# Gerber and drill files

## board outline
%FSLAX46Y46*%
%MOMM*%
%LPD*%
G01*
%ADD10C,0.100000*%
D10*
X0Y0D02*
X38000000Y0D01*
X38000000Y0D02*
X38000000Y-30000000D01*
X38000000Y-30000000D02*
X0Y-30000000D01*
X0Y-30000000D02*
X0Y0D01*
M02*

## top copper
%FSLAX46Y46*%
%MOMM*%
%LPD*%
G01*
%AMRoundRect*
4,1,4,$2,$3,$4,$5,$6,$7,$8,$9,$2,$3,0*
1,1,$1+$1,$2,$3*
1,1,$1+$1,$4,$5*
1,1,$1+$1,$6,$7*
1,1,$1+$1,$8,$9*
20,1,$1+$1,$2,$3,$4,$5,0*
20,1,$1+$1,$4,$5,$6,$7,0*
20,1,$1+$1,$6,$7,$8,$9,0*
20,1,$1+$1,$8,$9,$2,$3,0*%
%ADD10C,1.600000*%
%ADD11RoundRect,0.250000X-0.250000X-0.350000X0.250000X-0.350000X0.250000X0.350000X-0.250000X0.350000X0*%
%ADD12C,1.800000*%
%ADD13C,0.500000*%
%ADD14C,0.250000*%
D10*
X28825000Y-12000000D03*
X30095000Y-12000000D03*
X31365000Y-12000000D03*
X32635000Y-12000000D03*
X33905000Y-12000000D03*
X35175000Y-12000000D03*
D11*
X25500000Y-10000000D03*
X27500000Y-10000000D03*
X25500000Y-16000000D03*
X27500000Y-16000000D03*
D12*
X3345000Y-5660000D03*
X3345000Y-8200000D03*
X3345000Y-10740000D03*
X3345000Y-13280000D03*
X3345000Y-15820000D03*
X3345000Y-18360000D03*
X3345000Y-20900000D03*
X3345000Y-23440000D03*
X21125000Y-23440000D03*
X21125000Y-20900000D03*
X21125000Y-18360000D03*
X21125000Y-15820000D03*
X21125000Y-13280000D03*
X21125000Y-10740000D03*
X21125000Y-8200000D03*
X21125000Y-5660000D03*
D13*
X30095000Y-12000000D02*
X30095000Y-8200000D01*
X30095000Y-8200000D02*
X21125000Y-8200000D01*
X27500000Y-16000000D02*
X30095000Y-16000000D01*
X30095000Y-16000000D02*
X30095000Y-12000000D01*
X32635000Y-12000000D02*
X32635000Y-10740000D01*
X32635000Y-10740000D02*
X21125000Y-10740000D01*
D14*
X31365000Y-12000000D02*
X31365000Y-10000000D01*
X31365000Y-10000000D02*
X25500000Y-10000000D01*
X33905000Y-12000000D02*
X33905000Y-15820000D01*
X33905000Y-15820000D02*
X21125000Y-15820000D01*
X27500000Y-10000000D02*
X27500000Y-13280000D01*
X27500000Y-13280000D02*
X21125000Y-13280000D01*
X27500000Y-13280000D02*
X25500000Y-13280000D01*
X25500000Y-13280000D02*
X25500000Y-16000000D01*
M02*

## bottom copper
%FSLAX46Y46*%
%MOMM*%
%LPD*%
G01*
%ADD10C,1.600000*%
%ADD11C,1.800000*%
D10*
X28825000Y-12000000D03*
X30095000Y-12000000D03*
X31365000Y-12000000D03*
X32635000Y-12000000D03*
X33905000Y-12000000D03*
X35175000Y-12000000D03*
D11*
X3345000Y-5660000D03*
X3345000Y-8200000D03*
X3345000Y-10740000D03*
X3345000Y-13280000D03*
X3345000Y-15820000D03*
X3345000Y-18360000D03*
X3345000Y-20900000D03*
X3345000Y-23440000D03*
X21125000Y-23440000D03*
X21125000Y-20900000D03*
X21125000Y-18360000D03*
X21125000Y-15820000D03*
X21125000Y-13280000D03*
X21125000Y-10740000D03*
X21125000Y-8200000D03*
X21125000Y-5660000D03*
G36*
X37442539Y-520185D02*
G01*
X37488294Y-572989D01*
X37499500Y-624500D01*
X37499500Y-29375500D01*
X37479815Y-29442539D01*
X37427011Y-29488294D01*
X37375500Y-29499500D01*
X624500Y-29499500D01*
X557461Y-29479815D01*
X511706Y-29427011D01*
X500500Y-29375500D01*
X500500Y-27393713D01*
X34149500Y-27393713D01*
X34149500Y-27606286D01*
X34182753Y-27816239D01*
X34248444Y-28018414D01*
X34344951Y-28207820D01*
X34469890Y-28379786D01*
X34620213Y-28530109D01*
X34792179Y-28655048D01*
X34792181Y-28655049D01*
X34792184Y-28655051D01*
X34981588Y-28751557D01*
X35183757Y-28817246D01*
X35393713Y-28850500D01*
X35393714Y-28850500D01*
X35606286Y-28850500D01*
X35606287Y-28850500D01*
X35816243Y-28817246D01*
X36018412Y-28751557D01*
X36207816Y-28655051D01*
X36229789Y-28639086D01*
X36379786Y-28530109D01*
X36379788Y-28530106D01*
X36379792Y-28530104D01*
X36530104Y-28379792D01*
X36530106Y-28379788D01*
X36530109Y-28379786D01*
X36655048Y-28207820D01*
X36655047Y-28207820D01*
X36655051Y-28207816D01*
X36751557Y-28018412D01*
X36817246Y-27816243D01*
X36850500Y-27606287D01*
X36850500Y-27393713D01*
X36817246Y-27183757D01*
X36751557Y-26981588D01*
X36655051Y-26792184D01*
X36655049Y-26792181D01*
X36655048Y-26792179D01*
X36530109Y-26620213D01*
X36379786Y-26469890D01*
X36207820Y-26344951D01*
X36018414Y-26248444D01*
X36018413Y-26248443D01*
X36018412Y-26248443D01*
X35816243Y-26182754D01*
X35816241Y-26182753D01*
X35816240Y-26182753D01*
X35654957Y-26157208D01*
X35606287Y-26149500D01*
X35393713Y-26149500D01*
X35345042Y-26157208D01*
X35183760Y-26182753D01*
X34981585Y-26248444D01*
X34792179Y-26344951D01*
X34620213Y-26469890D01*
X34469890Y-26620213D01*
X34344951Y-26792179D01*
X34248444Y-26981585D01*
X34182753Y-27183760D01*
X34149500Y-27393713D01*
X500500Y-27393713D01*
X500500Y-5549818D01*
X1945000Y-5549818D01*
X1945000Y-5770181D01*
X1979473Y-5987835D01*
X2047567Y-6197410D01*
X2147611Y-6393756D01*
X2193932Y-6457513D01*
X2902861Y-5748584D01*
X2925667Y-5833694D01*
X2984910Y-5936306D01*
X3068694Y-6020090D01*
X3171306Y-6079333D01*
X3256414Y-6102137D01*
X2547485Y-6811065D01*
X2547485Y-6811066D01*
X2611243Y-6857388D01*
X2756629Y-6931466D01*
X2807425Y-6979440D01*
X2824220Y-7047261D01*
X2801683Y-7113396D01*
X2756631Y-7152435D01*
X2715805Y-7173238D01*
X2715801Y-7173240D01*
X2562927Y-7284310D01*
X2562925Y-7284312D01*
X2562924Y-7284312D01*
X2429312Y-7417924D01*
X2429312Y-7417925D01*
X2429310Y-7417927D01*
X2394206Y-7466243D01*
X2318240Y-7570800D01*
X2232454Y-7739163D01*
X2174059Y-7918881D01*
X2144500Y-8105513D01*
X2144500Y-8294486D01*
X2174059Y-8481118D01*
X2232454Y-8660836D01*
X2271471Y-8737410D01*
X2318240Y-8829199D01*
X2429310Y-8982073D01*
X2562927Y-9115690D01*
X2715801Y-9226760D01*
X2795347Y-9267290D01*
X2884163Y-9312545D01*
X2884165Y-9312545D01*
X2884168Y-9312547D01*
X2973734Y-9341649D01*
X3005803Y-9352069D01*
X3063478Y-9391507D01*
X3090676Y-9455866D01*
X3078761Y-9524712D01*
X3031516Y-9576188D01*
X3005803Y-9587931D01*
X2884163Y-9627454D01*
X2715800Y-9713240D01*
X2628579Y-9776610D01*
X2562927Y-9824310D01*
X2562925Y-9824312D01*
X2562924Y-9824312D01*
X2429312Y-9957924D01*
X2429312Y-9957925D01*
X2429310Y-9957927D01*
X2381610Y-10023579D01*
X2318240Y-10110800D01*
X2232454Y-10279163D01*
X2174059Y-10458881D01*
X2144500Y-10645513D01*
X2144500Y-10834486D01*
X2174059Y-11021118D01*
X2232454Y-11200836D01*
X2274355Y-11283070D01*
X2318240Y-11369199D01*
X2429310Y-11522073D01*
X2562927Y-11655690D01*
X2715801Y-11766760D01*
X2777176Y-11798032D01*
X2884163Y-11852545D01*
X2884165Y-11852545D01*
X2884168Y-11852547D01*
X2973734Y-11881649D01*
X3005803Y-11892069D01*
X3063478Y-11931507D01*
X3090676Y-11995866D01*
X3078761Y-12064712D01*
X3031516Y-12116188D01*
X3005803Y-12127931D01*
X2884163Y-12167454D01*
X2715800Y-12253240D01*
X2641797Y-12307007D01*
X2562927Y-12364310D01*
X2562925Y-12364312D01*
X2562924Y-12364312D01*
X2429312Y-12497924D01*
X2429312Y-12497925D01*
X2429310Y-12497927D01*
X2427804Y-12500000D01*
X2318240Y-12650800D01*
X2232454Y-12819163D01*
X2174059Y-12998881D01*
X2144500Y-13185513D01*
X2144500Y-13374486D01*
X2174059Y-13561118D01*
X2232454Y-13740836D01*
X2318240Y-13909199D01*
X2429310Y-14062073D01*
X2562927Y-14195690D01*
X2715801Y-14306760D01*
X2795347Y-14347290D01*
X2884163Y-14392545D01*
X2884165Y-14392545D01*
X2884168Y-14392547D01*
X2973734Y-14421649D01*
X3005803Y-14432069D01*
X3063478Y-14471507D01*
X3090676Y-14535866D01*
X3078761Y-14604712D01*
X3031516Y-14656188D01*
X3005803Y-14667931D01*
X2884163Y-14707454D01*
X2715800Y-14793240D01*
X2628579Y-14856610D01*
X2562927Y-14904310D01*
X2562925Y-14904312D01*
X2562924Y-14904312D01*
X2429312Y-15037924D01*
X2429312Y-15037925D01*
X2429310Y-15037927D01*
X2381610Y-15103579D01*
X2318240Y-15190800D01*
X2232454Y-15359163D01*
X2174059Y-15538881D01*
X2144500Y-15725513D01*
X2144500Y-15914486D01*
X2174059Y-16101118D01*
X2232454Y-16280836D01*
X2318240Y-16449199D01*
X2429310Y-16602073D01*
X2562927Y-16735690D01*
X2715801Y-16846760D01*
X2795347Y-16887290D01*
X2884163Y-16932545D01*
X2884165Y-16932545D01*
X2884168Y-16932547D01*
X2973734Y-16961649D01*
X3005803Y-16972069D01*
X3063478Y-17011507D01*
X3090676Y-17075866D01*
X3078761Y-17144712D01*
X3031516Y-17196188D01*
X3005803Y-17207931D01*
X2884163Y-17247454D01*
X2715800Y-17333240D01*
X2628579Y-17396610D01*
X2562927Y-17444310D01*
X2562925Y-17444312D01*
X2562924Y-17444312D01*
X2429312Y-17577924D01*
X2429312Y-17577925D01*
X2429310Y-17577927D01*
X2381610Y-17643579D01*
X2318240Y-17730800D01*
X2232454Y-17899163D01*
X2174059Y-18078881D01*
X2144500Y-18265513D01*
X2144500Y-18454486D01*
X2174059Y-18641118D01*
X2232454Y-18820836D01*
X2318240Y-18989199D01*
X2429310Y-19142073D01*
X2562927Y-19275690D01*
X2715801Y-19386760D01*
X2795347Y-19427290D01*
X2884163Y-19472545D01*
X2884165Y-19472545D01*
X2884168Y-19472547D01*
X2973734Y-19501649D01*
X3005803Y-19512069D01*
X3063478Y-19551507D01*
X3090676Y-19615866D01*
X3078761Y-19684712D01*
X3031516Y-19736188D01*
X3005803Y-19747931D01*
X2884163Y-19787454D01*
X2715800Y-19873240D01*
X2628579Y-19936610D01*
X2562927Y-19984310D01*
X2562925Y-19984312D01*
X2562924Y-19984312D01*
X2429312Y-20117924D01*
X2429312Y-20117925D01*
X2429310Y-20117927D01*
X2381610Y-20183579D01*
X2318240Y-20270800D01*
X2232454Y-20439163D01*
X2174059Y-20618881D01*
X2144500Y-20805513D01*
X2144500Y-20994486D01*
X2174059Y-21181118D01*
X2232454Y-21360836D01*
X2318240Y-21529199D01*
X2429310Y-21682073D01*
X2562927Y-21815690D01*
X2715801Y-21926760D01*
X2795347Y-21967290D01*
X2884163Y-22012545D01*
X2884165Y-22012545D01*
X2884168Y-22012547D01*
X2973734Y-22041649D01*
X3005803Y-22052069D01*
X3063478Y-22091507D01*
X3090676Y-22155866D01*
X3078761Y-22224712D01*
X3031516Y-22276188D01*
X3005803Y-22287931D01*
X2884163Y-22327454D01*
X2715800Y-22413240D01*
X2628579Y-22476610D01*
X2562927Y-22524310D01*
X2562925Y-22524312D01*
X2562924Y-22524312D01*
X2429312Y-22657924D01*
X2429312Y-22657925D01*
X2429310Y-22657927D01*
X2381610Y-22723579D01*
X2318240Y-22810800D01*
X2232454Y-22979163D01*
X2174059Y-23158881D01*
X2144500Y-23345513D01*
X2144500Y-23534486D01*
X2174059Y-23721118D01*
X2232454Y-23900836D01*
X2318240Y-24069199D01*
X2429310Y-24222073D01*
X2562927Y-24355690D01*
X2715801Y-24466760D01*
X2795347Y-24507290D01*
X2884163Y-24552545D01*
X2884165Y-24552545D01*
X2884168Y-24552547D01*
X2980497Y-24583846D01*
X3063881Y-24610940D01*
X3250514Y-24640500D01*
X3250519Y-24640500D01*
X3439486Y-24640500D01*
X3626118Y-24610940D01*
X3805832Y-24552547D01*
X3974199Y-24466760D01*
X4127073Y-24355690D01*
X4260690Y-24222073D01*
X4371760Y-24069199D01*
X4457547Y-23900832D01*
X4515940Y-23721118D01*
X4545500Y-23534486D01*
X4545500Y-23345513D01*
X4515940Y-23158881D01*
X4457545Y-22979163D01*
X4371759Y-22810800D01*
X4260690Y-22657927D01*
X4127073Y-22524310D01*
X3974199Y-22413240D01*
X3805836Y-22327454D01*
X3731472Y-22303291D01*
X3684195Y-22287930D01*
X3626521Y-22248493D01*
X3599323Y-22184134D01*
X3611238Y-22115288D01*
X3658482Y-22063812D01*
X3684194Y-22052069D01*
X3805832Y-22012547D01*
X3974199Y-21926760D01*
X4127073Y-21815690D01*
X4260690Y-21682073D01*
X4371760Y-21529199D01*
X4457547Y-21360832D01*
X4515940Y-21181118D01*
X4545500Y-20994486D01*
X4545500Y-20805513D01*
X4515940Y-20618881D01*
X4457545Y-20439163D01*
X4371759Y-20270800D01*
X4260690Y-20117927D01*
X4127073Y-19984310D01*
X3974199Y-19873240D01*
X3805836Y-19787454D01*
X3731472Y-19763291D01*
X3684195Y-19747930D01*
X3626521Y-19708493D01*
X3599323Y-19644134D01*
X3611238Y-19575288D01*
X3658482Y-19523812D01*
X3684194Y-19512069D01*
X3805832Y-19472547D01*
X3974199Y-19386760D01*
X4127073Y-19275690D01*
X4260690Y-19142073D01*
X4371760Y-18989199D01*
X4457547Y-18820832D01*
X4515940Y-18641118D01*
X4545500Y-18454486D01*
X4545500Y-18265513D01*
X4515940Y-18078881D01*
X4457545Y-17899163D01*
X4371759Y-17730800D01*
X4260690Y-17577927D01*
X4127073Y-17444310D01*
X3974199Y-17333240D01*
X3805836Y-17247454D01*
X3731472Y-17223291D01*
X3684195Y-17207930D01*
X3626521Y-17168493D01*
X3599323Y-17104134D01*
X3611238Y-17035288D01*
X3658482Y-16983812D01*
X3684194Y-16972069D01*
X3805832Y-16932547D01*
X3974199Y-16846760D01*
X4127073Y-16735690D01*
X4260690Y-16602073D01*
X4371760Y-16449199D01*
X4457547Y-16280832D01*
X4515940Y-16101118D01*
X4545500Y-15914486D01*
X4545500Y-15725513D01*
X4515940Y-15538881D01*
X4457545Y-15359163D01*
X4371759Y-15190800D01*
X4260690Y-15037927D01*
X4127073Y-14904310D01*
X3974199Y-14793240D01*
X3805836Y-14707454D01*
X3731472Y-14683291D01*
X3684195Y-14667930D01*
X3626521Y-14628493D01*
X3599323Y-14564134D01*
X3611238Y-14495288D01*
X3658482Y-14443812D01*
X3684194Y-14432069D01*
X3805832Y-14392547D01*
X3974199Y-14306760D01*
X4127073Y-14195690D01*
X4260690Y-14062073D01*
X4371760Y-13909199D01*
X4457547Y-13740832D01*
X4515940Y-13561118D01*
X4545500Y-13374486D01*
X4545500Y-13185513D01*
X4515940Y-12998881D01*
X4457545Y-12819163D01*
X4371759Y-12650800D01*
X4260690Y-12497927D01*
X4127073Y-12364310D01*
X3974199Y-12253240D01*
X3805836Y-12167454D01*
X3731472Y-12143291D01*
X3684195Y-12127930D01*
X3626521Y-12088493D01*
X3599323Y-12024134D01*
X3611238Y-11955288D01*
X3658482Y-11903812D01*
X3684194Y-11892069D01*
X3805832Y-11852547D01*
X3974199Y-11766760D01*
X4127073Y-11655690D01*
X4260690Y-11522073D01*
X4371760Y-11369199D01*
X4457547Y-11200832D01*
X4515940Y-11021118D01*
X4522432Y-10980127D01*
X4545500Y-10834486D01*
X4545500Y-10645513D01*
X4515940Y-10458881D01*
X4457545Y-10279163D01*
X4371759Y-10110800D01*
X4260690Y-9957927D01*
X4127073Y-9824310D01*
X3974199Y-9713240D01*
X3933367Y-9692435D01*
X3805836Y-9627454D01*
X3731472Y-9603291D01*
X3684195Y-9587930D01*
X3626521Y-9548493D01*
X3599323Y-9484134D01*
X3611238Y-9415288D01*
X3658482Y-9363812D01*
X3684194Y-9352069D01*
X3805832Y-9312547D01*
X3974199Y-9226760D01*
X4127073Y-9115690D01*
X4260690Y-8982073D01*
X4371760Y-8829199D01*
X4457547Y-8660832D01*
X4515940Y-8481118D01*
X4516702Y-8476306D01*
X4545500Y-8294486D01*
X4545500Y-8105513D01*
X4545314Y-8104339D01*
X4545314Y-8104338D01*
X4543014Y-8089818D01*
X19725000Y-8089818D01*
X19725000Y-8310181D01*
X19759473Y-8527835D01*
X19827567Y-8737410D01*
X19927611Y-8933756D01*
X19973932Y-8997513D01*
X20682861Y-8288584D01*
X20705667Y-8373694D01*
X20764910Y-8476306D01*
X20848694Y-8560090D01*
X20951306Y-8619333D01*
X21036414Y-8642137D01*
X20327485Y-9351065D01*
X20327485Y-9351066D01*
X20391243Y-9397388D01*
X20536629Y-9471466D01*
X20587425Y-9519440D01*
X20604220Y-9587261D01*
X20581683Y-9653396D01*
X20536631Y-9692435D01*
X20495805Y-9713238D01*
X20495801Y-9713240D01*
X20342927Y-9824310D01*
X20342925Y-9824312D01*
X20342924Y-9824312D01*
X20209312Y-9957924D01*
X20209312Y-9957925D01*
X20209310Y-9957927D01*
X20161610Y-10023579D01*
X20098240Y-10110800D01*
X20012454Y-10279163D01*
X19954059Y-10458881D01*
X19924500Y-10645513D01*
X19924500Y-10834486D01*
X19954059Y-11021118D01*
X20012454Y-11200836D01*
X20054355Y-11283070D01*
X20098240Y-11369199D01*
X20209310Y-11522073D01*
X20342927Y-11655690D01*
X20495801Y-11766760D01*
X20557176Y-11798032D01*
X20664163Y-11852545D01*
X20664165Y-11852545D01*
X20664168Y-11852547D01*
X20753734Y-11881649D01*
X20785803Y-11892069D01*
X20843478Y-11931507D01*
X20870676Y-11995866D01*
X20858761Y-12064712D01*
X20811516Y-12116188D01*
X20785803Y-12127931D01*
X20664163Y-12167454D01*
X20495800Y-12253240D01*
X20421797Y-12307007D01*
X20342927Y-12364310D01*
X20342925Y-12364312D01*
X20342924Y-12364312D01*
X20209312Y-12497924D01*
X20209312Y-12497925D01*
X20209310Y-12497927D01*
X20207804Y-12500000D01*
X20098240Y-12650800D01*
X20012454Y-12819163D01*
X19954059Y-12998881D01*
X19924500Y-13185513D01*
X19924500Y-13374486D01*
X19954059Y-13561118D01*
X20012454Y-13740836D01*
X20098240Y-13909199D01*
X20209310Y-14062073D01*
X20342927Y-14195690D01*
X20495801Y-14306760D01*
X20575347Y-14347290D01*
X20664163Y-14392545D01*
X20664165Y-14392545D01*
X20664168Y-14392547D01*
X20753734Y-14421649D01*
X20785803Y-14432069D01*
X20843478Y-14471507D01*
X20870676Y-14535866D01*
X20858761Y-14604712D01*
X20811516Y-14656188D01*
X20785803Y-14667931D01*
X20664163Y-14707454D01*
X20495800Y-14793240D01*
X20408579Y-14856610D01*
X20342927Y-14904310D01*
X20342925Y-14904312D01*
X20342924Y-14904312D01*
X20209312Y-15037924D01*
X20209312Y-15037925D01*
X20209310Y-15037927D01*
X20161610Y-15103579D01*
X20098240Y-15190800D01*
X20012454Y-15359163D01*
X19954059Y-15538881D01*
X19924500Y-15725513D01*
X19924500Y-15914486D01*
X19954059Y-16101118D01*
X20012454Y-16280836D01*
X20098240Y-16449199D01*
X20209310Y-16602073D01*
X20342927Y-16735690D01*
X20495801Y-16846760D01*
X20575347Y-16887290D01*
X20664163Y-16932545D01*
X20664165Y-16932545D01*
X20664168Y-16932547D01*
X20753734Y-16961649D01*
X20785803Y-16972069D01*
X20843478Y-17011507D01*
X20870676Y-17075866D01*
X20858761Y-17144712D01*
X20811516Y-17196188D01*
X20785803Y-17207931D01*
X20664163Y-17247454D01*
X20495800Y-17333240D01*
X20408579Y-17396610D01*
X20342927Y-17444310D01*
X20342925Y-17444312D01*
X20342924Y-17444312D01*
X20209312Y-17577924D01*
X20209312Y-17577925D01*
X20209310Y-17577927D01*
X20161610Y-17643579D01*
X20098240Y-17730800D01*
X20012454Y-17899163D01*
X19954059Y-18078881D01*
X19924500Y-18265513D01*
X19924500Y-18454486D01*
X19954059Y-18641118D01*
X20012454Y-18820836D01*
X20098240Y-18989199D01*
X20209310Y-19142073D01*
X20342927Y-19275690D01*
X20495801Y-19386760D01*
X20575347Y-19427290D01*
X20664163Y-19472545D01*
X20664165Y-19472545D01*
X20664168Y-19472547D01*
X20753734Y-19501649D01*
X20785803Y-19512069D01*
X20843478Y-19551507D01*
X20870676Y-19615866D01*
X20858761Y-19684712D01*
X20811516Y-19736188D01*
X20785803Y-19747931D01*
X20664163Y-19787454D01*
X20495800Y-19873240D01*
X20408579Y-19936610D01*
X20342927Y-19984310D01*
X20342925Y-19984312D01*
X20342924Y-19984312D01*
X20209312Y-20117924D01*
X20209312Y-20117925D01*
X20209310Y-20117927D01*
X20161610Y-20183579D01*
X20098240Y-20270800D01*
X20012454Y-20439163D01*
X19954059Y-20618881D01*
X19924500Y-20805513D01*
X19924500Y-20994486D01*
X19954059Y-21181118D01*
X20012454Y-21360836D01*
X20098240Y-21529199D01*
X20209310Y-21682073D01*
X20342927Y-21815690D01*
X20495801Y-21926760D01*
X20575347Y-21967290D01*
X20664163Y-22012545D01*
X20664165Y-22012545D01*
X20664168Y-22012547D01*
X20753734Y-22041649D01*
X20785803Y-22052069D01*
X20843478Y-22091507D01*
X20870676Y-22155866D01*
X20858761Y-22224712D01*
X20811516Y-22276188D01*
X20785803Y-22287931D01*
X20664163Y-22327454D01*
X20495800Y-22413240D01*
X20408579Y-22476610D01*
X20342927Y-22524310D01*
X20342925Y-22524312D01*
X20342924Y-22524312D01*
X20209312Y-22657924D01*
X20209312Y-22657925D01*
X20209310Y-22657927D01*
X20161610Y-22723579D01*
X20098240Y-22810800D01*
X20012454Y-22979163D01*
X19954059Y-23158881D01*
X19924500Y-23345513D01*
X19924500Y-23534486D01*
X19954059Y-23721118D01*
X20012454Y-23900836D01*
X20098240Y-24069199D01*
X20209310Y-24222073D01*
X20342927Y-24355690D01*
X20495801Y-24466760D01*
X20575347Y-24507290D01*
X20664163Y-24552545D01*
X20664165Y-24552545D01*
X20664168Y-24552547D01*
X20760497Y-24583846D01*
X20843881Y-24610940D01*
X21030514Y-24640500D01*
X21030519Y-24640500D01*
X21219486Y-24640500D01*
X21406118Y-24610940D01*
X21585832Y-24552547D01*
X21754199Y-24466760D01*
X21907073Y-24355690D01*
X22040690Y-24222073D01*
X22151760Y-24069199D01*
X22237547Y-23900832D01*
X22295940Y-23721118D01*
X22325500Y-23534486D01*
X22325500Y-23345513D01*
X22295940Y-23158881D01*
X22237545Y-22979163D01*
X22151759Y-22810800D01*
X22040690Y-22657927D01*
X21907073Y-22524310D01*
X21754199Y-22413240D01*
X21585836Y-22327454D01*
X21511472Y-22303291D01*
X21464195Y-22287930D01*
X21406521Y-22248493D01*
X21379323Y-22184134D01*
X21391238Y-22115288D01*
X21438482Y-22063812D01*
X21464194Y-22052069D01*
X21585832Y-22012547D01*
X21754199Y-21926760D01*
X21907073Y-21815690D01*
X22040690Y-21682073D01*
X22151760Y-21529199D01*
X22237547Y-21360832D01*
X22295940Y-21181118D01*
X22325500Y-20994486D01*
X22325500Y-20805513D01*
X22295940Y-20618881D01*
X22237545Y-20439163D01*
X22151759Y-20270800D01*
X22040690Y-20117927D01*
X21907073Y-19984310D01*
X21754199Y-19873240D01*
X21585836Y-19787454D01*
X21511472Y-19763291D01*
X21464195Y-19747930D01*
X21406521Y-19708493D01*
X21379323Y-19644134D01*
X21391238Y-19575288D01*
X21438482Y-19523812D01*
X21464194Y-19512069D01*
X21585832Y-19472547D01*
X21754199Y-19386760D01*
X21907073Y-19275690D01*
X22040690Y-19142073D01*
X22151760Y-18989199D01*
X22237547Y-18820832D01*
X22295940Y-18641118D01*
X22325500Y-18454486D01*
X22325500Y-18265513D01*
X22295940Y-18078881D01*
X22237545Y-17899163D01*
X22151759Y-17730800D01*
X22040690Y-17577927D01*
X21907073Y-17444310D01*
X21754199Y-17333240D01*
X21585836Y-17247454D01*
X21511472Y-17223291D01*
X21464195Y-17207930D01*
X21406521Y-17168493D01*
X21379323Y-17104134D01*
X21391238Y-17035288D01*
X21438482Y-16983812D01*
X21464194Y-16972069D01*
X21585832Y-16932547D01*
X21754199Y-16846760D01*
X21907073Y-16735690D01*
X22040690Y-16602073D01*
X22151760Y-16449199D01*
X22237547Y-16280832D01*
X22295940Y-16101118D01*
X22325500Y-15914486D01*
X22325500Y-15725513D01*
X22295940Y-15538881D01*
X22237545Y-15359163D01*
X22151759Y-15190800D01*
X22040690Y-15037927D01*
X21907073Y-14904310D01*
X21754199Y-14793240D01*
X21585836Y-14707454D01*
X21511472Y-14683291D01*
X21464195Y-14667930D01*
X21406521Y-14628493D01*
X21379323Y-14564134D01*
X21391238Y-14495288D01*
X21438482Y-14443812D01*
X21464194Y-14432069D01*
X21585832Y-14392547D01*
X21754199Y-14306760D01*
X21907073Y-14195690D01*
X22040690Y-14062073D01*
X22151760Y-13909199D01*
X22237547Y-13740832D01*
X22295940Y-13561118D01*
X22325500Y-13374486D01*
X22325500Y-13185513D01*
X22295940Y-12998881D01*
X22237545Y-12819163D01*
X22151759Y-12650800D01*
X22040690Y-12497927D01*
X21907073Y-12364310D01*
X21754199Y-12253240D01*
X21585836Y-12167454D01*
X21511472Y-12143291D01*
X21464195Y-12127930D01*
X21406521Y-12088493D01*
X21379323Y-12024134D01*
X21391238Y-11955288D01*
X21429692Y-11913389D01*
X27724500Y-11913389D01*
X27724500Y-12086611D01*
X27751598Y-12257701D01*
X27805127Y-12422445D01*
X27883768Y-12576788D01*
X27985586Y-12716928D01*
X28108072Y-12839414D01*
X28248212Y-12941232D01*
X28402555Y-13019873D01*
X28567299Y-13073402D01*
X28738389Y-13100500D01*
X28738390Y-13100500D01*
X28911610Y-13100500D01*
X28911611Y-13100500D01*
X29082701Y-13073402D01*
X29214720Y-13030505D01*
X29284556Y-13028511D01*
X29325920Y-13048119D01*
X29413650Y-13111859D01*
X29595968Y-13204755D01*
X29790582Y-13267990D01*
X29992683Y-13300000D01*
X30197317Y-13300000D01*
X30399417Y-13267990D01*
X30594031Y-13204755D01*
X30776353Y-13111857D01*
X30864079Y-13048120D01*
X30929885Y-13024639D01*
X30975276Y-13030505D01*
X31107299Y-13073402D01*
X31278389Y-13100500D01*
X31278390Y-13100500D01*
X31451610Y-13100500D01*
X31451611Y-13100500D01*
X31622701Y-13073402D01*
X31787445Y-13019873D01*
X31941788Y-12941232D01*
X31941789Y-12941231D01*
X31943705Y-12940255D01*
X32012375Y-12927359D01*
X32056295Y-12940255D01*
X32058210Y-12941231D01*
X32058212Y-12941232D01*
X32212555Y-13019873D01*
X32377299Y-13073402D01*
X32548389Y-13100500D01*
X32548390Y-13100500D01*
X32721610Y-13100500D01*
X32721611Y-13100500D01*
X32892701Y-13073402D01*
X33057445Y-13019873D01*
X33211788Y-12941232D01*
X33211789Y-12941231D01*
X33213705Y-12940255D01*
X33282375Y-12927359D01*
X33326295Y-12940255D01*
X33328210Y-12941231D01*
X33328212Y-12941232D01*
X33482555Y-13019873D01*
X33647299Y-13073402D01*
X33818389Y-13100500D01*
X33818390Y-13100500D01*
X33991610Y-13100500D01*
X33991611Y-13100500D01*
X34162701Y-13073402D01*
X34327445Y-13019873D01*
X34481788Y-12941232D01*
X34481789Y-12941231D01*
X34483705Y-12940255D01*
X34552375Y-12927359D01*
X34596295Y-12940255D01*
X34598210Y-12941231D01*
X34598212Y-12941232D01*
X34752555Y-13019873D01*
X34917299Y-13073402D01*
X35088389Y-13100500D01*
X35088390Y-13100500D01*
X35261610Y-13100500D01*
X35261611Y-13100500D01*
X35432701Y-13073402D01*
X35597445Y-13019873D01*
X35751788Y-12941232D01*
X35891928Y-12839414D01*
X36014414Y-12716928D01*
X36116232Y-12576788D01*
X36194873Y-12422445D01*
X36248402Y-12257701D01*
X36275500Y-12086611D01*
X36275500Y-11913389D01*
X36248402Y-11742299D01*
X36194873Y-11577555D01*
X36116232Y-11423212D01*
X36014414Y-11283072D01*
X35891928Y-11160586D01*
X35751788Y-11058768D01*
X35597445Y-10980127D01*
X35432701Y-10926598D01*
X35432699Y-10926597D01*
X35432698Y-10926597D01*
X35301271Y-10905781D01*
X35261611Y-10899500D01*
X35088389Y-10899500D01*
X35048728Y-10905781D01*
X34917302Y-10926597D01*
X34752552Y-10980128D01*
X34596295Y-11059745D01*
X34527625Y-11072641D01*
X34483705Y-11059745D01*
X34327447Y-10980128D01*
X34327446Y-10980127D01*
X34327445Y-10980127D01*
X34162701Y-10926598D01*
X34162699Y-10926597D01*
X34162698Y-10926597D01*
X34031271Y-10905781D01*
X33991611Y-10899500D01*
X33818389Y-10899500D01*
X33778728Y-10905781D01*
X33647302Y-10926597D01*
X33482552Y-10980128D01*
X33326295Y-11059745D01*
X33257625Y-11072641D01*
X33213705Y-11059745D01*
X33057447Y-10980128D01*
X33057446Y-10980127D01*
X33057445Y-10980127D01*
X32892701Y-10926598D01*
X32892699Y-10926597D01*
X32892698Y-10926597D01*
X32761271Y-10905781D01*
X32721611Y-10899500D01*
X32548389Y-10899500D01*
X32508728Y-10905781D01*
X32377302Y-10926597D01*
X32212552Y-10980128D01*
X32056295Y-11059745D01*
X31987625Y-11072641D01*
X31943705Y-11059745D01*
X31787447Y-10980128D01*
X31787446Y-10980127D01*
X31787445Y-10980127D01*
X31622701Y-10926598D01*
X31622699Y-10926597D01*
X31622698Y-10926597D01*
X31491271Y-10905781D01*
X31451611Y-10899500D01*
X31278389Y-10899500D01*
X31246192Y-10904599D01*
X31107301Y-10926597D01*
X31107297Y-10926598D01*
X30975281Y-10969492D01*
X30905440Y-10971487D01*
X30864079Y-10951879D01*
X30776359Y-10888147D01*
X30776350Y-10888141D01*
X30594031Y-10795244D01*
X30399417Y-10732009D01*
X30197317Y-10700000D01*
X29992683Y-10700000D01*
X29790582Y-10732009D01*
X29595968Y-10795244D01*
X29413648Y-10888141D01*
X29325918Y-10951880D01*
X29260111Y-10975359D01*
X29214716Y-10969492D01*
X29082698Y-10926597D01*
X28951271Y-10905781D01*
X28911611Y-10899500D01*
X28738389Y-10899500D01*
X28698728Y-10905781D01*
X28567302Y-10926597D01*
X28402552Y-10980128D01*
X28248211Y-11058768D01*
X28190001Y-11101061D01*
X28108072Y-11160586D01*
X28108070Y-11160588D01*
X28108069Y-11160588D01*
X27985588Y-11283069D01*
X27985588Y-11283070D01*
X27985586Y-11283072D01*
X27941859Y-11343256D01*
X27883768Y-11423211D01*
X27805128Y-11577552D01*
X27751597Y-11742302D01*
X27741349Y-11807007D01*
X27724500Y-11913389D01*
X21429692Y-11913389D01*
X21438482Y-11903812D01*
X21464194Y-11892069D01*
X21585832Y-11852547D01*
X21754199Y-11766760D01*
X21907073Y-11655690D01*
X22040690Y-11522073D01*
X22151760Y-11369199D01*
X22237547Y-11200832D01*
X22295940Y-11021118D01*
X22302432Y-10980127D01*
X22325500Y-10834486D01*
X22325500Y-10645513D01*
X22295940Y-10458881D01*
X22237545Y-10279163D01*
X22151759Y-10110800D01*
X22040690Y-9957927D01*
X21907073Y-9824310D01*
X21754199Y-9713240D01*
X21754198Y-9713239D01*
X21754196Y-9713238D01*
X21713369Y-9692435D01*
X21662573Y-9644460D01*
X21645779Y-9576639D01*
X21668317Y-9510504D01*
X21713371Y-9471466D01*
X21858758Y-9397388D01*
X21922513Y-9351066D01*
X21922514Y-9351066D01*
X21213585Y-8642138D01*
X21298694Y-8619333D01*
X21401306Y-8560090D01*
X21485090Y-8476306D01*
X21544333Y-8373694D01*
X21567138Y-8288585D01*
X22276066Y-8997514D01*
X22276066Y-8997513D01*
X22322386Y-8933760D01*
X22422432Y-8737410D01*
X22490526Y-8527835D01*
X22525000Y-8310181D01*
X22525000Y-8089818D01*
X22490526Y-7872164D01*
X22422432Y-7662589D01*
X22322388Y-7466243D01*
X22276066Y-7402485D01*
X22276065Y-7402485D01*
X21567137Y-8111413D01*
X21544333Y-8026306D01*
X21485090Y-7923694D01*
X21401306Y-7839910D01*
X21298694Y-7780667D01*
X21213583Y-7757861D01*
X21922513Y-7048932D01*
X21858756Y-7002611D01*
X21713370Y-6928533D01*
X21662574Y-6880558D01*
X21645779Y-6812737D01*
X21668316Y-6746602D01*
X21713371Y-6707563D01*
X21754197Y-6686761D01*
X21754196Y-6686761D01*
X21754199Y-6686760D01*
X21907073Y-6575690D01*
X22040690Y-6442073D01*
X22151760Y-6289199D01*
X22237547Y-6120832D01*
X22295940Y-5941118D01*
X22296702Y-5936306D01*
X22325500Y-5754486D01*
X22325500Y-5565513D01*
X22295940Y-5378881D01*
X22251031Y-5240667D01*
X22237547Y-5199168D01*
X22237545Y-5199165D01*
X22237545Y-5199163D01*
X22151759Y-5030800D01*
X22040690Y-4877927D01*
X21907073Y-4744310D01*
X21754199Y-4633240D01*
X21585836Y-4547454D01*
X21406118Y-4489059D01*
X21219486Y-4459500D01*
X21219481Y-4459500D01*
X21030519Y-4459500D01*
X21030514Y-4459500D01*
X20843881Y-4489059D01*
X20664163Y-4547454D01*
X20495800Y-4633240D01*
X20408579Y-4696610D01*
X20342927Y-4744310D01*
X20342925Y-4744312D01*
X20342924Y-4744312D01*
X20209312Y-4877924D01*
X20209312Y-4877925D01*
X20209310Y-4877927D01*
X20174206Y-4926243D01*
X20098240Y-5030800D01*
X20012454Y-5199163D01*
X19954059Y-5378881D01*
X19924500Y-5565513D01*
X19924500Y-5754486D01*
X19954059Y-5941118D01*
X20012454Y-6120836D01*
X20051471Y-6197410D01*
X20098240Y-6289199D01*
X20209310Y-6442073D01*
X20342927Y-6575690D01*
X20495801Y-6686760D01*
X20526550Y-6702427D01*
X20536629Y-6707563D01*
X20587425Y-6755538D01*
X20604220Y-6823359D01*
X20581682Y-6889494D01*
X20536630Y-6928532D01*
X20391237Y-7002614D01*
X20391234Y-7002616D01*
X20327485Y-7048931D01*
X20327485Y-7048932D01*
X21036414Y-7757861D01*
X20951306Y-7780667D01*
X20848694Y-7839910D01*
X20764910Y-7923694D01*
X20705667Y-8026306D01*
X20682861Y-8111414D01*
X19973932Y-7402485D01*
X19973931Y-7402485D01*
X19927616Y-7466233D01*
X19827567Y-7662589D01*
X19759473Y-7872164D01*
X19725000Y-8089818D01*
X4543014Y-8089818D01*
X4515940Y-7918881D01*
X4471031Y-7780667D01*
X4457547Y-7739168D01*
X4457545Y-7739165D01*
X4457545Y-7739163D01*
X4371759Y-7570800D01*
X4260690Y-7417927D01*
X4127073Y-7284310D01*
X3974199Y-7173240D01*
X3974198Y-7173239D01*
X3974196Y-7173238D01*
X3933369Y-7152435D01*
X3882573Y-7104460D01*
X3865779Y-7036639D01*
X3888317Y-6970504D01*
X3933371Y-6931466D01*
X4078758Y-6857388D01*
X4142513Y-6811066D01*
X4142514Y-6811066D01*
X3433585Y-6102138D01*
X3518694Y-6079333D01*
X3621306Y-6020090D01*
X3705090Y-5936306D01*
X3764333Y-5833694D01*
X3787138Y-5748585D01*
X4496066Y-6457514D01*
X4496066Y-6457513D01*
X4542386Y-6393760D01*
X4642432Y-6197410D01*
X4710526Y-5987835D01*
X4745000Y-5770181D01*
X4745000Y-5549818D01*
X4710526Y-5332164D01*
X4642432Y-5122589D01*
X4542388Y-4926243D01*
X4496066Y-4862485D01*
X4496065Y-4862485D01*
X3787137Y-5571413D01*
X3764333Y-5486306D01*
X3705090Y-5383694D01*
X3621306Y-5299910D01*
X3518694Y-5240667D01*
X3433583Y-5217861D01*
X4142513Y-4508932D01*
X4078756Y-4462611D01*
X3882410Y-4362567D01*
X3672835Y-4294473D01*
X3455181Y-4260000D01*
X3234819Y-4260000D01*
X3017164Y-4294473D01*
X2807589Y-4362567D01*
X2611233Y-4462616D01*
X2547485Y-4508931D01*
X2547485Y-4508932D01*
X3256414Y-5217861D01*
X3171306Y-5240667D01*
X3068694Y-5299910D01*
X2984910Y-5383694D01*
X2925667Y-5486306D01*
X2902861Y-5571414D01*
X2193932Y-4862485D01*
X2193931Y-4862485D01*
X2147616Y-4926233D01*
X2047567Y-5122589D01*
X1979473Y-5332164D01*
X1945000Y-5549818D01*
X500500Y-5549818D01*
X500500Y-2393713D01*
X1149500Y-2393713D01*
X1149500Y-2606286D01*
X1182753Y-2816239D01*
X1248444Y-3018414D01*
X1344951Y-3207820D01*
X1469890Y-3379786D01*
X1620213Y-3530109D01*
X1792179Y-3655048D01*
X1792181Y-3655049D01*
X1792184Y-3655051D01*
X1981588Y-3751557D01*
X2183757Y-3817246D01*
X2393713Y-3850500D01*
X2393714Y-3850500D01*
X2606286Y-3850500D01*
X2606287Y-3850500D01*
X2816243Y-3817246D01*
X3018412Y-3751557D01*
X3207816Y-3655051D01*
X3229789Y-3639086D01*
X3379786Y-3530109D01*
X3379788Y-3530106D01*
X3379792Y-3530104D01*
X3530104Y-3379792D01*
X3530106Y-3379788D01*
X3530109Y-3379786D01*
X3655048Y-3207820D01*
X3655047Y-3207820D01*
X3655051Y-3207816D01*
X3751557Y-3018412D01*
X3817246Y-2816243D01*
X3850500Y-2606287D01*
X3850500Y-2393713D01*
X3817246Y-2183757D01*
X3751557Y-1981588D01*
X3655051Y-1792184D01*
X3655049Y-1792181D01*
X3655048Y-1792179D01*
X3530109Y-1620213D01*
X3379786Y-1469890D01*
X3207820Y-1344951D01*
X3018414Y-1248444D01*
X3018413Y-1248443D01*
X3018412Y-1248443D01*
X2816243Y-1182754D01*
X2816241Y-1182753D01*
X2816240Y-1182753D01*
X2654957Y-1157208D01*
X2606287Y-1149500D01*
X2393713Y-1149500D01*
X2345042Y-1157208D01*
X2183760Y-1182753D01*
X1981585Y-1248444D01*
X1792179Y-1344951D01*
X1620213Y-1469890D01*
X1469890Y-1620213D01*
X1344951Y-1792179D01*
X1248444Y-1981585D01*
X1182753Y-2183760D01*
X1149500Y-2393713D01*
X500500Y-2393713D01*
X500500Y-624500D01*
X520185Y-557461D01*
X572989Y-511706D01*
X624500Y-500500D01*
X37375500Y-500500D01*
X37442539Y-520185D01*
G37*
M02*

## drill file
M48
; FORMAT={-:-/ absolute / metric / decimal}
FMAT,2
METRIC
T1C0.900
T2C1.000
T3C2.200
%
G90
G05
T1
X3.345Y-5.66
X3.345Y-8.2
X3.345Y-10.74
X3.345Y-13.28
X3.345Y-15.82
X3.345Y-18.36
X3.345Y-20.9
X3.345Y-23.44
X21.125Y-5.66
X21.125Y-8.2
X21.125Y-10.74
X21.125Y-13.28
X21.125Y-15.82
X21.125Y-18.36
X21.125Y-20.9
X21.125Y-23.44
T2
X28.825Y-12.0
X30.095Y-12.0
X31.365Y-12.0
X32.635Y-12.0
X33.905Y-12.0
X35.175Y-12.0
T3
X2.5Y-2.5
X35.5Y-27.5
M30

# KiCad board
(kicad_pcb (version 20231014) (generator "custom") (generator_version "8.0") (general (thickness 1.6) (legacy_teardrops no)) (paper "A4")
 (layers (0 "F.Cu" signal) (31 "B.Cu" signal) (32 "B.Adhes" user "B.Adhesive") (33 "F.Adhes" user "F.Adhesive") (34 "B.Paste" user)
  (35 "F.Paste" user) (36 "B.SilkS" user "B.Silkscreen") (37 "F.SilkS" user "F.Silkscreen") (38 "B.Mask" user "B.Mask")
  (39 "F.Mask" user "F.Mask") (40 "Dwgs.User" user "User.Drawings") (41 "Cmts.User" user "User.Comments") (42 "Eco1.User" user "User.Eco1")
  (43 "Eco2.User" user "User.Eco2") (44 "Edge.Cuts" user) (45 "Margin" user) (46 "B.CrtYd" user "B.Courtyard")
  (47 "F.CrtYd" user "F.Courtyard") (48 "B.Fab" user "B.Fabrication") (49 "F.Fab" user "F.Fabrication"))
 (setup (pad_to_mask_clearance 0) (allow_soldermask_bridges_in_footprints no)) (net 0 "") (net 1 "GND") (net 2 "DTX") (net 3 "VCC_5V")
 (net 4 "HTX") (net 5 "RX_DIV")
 (gr_line (start 0 0) (end 38 0) (stroke (width 0.1) (type solid)) (layer "Edge.Cuts"))
 (gr_line (start 38 0) (end 38 30) (stroke (width 0.1) (type solid)) (layer "Edge.Cuts"))
 (gr_line (start 38 30) (end 0 30) (stroke (width 0.1) (type solid)) (layer "Edge.Cuts"))
 (gr_line (start 0 30) (end 0 0) (stroke (width 0.1) (type solid)) (layer "Edge.Cuts"))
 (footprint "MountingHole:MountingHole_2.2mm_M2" (layer "F.Cu") (at 2.5 2.5)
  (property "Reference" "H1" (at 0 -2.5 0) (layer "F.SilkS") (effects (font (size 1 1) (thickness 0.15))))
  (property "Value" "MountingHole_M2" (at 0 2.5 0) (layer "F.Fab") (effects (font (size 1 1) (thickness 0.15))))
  (pad "" np_thru_hole circle (at 0 0) (size 2.2 2.2) (drill 2.2) (layers "*.Cu" "*.Mask")))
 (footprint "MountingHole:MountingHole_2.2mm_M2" (layer "F.Cu") (at 35.5 27.5)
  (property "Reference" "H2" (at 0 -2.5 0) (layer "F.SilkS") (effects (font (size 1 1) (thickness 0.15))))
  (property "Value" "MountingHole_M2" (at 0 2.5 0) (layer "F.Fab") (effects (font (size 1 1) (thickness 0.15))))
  (pad "" np_thru_hole circle (at 0 0) (size 2.2 2.2) (drill 2.2) (layers "*.Cu" "*.Mask")))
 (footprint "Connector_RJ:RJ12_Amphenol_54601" (layer "F.Cu") (at 32 12)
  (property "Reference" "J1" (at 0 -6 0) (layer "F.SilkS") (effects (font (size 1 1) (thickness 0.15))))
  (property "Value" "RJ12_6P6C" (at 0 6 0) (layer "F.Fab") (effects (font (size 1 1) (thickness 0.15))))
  (pad "1" thru_hole circle (at -3.175 0) (size 1.6 1.6) (drill 1.0) (layers "*.Cu" "*.Mask") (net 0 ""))
  (pad "2" thru_hole circle (at -1.905 0) (size 1.6 1.6) (drill 1.0) (layers "*.Cu" "*.Mask") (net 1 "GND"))
  (pad "3" thru_hole circle (at -0.635 0) (size 1.6 1.6) (drill 1.0) (layers "*.Cu" "*.Mask") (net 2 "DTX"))
  (pad "4" thru_hole circle (at 0.635 0) (size 1.6 1.6) (drill 1.0) (layers "*.Cu" "*.Mask") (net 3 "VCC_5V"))
  (pad "5" thru_hole circle (at 1.905 0) (size 1.6 1.6) (drill 1.0) (layers "*.Cu" "*.Mask") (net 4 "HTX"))
  (pad "6" thru_hole circle (at 3.175 0) (size 1.6 1.6) (drill 1.0) (layers "*.Cu" "*.Mask") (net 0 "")))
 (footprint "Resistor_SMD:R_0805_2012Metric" (layer "F.Cu") (at 26.5 10)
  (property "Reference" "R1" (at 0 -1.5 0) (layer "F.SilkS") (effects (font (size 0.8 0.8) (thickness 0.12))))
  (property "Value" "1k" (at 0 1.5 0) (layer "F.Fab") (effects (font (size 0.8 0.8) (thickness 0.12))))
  (pad "1" smd roundrect (at -1 0) (size 1.0 1.2) (layers "F.Cu" "F.Paste" "F.Mask") (roundrect_rratio 0.25) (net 2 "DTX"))
  (pad "2" smd roundrect (at 1 0) (size 1.0 1.2) (layers "F.Cu" "F.Paste" "F.Mask") (roundrect_rratio 0.25) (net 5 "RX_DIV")))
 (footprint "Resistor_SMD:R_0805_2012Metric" (layer "F.Cu") (at 26.5 16)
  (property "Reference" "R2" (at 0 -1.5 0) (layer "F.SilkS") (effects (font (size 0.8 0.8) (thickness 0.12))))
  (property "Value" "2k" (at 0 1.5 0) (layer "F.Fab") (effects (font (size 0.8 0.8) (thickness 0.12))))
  (pad "1" smd roundrect (at -1 0) (size 1.0 1.2) (layers "F.Cu" "F.Paste" "F.Mask") (roundrect_rratio 0.25) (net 5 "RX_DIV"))
  (pad "2" smd roundrect (at 1 0) (size 1.0 1.2) (layers "F.Cu" "F.Paste" "F.Mask") (roundrect_rratio 0.25) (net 1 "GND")))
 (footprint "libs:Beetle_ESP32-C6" (layer "F.Cu") (at 2 28)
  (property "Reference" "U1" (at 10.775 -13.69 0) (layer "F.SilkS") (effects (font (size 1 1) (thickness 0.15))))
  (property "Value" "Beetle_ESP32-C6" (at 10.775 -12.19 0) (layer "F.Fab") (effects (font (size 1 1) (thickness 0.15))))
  (pad "1" thru_hole circle (at 1.345 -22.34) (size 1.8 1.8) (drill 0.9) (layers "*.Cu" "*.Mask") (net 1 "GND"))
  (pad "2" thru_hole circle (at 1.345 -19.8) (size 1.8 1.8) (drill 0.9) (layers "*.Cu" "*.Mask") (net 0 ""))
  (pad "3" thru_hole circle (at 1.345 -17.26) (size 1.8 1.8) (drill 0.9) (layers "*.Cu" "*.Mask") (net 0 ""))
  (pad "4" thru_hole circle (at 1.345 -14.72) (size 1.8 1.8) (drill 0.9) (layers "*.Cu" "*.Mask") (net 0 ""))
  (pad "5" thru_hole circle (at 1.345 -12.18) (size 1.8 1.8) (drill 0.9) (layers "*.Cu" "*.Mask") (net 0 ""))
  (pad "6" thru_hole circle (at 1.345 -9.64) (size 1.8 1.8) (drill 0.9) (layers "*.Cu" "*.Mask") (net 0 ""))
  (pad "7" thru_hole circle (at 1.345 -7.1) (size 1.8 1.8) (drill 0.9) (layers "*.Cu" "*.Mask") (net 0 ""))
  (pad "8" thru_hole circle (at 1.345 -4.56) (size 1.8 1.8) (drill 0.9) (layers "*.Cu" "*.Mask") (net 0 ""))
  (pad "9" thru_hole circle (at 19.125 -4.56) (size 1.8 1.8) (drill 0.9) (layers "*.Cu" "*.Mask") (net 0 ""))
  (pad "10" thru_hole circle (at 19.125 -7.1) (size 1.8 1.8) (drill 0.9) (layers "*.Cu" "*.Mask") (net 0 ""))
  (pad "11" thru_hole circle (at 19.125 -9.64) (size 1.8 1.8) (drill 0.9) (layers "*.Cu" "*.Mask") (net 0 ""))
  (pad "12" thru_hole circle (at 19.125 -12.18) (size 1.8 1.8) (drill 0.9) (layers "*.Cu" "*.Mask") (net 4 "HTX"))
  (pad "13" thru_hole circle (at 19.125 -14.72) (size 1.8 1.8) (drill 0.9) (layers "*.Cu" "*.Mask") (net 5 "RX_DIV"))
  (pad "14" thru_hole circle (at 19.125 -17.26) (size 1.8 1.8) (drill 0.9) (layers "*.Cu" "*.Mask") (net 3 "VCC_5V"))
  (pad "15" thru_hole circle (at 19.125 -19.8) (size 1.8 1.8) (drill 0.9) (layers "*.Cu" "*.Mask") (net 1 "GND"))
  (pad "16" thru_hole circle (at 19.125 -22.34) (size 1.8 1.8) (drill 0.9) (layers "*.Cu" "*.Mask") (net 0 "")))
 (segment (start 30.095 12) (end 30.095 8.2) (width 0.5) (layer "F.Cu") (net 1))
 (segment (start 30.095 8.2) (end 21.125 8.2) (width 0.5) (layer "F.Cu") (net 1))
 (segment (start 27.5 16) (end 30.095 16) (width 0.5) (layer "F.Cu") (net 1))
 (segment (start 30.095 16) (end 30.095 12) (width 0.5) (layer "F.Cu") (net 1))
 (segment (start 32.635 12) (end 32.635 10.74) (width 0.5) (layer "F.Cu") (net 3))
 (segment (start 32.635 10.74) (end 21.125 10.74) (width 0.5) (layer "F.Cu") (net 3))
 (segment (start 31.365 12) (end 31.365 10) (width 0.25) (layer "F.Cu") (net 2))
 (segment (start 31.365 10) (end 25.5 10) (width 0.25) (layer "F.Cu") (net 2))
 (segment (start 33.905 12) (end 33.905 15.82) (width 0.25) (layer "F.Cu") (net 4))
 (segment (start 33.905 15.82) (end 21.125 15.82) (width 0.25) (layer "F.Cu") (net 4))
 (segment (start 27.5 10) (end 27.5 13.28) (width 0.25) (layer "F.Cu") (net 5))
 (segment (start 27.5 13.28) (end 21.125 13.28) (width 0.25) (layer "F.Cu") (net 5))
 (segment (start 27.5 13.28) (end 25.5 13.28) (width 0.25) (layer "F.Cu") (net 5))
 (segment (start 25.5 13.28) (end 25.5 16) (width 0.25) (layer "F.Cu") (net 5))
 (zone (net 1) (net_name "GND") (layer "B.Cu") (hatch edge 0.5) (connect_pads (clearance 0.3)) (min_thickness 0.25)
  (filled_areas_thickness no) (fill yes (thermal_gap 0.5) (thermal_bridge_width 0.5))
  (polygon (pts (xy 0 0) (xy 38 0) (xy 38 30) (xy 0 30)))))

